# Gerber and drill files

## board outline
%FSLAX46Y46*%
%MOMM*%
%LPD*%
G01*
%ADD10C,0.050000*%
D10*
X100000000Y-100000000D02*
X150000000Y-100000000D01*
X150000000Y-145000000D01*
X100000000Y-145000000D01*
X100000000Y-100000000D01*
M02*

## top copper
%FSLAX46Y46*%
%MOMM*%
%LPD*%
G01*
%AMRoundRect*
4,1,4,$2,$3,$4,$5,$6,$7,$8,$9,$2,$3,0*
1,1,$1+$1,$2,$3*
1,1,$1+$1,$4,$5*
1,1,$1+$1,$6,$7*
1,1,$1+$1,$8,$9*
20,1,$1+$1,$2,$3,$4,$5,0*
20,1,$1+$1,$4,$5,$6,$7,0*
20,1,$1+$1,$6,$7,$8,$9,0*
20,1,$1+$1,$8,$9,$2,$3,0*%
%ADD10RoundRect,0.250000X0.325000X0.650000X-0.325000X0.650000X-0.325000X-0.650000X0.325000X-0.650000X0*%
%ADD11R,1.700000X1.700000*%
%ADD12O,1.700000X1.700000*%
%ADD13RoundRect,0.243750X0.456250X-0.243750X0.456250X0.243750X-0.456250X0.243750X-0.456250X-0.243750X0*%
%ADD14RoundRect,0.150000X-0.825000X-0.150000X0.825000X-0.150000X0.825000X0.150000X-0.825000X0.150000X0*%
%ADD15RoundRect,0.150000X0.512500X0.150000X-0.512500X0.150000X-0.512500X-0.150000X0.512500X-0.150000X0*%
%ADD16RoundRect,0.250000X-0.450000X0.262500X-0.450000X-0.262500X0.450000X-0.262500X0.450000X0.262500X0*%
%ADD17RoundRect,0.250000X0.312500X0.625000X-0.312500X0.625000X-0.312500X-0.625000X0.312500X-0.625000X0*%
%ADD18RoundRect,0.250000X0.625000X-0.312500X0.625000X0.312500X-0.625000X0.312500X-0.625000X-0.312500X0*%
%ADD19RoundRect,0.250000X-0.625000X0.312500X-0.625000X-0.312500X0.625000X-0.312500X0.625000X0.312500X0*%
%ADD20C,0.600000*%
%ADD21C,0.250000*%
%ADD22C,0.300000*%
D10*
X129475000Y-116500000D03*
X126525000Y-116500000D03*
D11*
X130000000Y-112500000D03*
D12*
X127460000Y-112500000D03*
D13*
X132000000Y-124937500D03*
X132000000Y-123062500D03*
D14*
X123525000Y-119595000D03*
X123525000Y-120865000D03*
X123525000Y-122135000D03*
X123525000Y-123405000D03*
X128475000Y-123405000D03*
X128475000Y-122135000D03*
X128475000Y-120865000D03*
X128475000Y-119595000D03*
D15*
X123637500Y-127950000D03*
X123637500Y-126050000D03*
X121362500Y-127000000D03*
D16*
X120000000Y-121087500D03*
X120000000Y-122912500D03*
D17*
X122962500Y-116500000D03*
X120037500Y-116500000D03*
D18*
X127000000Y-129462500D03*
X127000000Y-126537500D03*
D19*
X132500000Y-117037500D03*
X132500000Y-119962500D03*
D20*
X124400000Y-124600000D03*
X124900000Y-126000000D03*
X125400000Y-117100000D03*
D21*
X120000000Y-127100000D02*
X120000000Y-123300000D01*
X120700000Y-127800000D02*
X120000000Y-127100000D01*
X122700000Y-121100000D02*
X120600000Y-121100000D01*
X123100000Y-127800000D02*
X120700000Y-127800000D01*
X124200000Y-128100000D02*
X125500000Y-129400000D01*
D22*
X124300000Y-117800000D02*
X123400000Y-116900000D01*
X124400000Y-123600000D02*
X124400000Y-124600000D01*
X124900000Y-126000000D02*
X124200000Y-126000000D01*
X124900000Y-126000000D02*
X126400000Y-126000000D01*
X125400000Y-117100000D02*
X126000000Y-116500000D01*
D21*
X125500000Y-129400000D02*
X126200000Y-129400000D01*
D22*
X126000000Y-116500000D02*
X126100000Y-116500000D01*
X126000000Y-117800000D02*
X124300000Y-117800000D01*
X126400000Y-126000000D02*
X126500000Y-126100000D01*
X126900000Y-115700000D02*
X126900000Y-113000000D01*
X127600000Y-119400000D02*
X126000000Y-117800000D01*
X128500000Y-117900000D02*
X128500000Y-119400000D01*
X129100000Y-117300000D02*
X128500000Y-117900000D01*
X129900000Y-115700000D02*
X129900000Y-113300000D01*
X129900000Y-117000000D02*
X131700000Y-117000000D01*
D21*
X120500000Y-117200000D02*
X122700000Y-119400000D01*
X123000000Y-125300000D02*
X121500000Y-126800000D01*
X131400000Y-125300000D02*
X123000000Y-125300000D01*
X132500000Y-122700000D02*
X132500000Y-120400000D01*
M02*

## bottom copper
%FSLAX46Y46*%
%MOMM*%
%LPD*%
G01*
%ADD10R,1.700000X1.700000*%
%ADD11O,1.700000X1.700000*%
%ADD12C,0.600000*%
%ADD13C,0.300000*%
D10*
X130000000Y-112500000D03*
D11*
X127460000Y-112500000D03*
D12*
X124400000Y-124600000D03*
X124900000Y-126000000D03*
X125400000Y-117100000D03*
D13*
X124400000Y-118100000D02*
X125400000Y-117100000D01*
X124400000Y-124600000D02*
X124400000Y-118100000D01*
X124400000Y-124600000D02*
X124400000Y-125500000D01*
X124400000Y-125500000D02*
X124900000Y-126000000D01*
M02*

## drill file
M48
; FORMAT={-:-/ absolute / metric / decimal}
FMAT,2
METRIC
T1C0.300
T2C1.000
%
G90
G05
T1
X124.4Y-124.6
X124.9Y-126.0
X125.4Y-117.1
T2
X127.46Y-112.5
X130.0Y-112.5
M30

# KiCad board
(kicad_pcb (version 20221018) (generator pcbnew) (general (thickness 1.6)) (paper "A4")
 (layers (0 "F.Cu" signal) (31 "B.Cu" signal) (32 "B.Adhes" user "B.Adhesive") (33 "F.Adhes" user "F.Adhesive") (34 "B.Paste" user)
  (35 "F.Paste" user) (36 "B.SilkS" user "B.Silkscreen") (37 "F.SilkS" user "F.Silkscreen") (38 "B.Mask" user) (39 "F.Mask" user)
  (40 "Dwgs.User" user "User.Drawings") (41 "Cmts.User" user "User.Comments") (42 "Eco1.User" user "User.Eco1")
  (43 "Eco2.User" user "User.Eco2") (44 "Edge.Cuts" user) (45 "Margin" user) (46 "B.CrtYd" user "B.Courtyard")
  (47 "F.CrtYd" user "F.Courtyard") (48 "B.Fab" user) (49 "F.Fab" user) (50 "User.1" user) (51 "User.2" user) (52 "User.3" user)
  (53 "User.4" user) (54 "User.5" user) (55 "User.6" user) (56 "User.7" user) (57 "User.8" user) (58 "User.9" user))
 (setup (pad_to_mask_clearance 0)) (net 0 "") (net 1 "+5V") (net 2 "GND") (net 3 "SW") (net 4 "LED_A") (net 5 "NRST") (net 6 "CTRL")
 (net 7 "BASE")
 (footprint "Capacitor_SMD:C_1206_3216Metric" (layer "F.Cu") (at 128 116.5 180)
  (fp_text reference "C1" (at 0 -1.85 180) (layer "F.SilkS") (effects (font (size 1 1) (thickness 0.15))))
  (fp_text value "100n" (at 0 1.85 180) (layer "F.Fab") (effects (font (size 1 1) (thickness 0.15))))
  (pad "1" smd roundrect (at -1.475 0 180) (size 1.15 1.8) (layers "F.Cu" "F.Paste" "F.Mask") (roundrect_rratio 0.217391) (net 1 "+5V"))
  (pad "2" smd roundrect (at 1.475 0 180) (size 1.15 1.8) (layers "F.Cu" "F.Paste" "F.Mask") (roundrect_rratio 0.217391) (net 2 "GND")))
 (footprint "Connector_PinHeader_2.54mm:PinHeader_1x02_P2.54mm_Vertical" (layer "F.Cu") (at 130 112.5 -90)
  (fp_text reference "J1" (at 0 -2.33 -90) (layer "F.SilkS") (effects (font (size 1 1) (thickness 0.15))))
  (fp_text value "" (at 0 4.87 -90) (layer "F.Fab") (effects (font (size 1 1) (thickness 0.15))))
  (pad "1" thru_hole rect (at 0 0 270) (size 1.7 1.7) (drill 1) (layers "*.Cu" "*.Mask") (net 1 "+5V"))
  (pad "2" thru_hole oval (at 0 2.54 270) (size 1.7 1.7) (drill 1) (layers "*.Cu" "*.Mask") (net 2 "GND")))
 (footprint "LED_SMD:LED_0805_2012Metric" (layer "F.Cu") (at 132 124 90)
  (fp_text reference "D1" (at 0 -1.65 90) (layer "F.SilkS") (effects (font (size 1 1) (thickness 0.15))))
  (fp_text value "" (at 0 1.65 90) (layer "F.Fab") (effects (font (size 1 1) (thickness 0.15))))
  (pad "1" smd roundrect (at -0.9375 0 90) (size 0.975 1.4) (layers "F.Cu" "F.Paste" "F.Mask") (roundrect_rratio 0.25) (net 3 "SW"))
  (pad "2" smd roundrect (at 0.9375 0 90) (size 0.975 1.4) (layers "F.Cu" "F.Paste" "F.Mask") (roundrect_rratio 0.25) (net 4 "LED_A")))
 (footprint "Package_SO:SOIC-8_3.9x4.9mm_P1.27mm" (layer "F.Cu") (at 126 121.5)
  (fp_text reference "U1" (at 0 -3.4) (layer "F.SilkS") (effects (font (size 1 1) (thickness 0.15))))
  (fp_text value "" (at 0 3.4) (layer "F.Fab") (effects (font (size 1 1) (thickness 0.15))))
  (pad "1" smd roundrect (at -2.475 -1.905) (size 1.95 0.6) (layers "F.Cu" "F.Paste" "F.Mask") (roundrect_rratio 0.25) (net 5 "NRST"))
  (pad "2" smd roundrect (at -2.475 -0.635) (size 1.95 0.6) (layers "F.Cu" "F.Paste" "F.Mask") (roundrect_rratio 0.25) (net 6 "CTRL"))
  (pad "3" smd roundrect (at -2.475 0.635) (size 1.95 0.6) (layers "F.Cu" "F.Paste" "F.Mask") (roundrect_rratio 0.25))
  (pad "4" smd roundrect (at -2.475 1.905) (size 1.95 0.6) (layers "F.Cu" "F.Paste" "F.Mask") (roundrect_rratio 0.25) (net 2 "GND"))
  (pad "5" smd roundrect (at 2.475 1.905) (size 1.95 0.6) (layers "F.Cu" "F.Paste" "F.Mask") (roundrect_rratio 0.25))
  (pad "6" smd roundrect (at 2.475 0.635) (size 1.95 0.6) (layers "F.Cu" "F.Paste" "F.Mask") (roundrect_rratio 0.25))
  (pad "7" smd roundrect (at 2.475 -0.635) (size 1.95 0.6) (layers "F.Cu" "F.Paste" "F.Mask") (roundrect_rratio 0.25))
  (pad "8" smd roundrect (at 2.475 -1.905) (size 1.95 0.6) (layers "F.Cu" "F.Paste" "F.Mask") (roundrect_rratio 0.25) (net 1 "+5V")))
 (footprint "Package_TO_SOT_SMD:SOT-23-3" (layer "F.Cu") (at 122.5 127 180)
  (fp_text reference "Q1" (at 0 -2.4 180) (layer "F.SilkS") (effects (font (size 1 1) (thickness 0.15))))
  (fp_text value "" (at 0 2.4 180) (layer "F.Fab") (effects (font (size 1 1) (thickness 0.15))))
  (pad "1" smd roundrect (at -1.1375 -0.95 180) (size 1.325 0.6) (layers "F.Cu" "F.Paste" "F.Mask") (roundrect_rratio 0.25) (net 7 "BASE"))
  (pad "2" smd roundrect (at -1.1375 0.95 180) (size 1.325 0.6) (layers "F.Cu" "F.Paste" "F.Mask") (roundrect_rratio 0.25) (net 2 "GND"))
  (pad "3" smd roundrect (at 1.1375 0 180) (size 1.325 0.6) (layers "F.Cu" "F.Paste" "F.Mask") (roundrect_rratio 0.25) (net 3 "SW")))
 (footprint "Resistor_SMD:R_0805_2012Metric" (layer "F.Cu") (at 120 122 -90)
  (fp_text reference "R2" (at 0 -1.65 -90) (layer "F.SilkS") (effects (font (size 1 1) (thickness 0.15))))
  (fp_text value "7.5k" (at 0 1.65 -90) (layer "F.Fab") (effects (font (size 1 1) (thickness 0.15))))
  (pad "1" smd roundrect (at -0.9125 0 270) (size 1.025 1.4) (layers "F.Cu" "F.Paste" "F.Mask") (roundrect_rratio 0.243902) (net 6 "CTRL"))
  (pad "2" smd roundrect (at 0.9125 0 270) (size 1.025 1.4) (layers "F.Cu" "F.Paste" "F.Mask") (roundrect_rratio 0.243902) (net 7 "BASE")))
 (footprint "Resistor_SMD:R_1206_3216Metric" (layer "F.Cu") (at 121.5 116.5 180)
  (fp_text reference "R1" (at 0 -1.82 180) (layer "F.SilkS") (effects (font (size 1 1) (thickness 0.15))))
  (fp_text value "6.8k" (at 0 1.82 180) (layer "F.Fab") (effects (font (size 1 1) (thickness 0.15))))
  (pad "1" smd roundrect (at -1.4625 0 180) (size 1.125 1.75) (layers "F.Cu" "F.Paste" "F.Mask") (roundrect_rratio 0.222222) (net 1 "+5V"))
  (pad "2" smd roundrect (at 1.4625 0 180) (size 1.125 1.75) (layers "F.Cu" "F.Paste" "F.Mask") (roundrect_rratio 0.222222) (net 5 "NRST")))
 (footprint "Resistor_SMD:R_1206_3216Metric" (layer "F.Cu") (at 127 128 90)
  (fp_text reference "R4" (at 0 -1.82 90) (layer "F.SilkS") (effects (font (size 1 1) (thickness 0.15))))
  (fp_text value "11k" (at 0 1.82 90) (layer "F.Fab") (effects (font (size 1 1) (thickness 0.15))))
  (pad "1" smd roundrect (at -1.4625 0 90) (size 1.125 1.75) (layers "F.Cu" "F.Paste" "F.Mask") (roundrect_rratio 0.222222) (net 7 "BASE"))
  (pad "2" smd roundrect (at 1.4625 0 90) (size 1.125 1.75) (layers "F.Cu" "F.Paste" "F.Mask") (roundrect_rratio 0.222222) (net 2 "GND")))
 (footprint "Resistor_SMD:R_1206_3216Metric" (layer "F.Cu") (at 132.5 118.5 -90)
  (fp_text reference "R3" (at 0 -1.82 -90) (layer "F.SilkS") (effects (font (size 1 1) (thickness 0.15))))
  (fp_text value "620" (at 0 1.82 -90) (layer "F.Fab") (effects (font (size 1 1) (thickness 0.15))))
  (pad "1" smd roundrect (at -1.4625 0 270) (size 1.125 1.75) (layers "F.Cu" "F.Paste" "F.Mask") (roundrect_rratio 0.222222) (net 1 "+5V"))
  (pad "2" smd roundrect (at 1.4625 0 270) (size 1.125 1.75) (layers "F.Cu" "F.Paste" "F.Mask") (roundrect_rratio 0.222222) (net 4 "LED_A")))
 (gr_rect (start 100 100) (end 150 145) (stroke (width 0.05) (type default)) (fill none) (layer "Edge.Cuts"))
 (segment (start 120 127.1) (end 120 123.3) (width 0.25) (layer "F.Cu") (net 7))
 (segment (start 120.7 127.8) (end 120 127.1) (width 0.25) (layer "F.Cu") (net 7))
 (segment (start 122.7 121.1) (end 120.6 121.1) (width 0.25) (layer "F.Cu") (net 6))
 (segment (start 123.1 127.8) (end 120.7 127.8) (width 0.25) (layer "F.Cu") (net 7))
 (segment (start 124.2 128.1) (end 125.5 129.4) (width 0.25) (layer "F.Cu") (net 7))
 (segment (start 124.3 117.8) (end 123.4 116.9) (width 0.3) (layer "F.Cu") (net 1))
 (segment (start 124.4 123.6) (end 124.4 124.6) (width 0.3) (layer "F.Cu") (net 2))
 (segment (start 124.9 126) (end 124.2 126) (width 0.3) (layer "F.Cu") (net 2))
 (segment (start 124.9 126) (end 126.4 126) (width 0.3) (layer "F.Cu") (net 2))
 (segment (start 125.4 117.1) (end 126 116.5) (width 0.3) (layer "F.Cu") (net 2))
 (segment (start 125.5 129.4) (end 126.2 129.4) (width 0.25) (layer "F.Cu") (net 7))
 (segment (start 126 116.5) (end 126.1 116.5) (width 0.3) (layer "F.Cu") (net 2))
 (segment (start 126 117.8) (end 124.3 117.8) (width 0.3) (layer "F.Cu") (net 1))
 (segment (start 126.4 126) (end 126.5 126.1) (width 0.3) (layer "F.Cu") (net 2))
 (segment (start 126.9 115.7) (end 126.9 113) (width 0.3) (layer "F.Cu") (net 2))
 (segment (start 127.6 119.4) (end 126 117.8) (width 0.3) (layer "F.Cu") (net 1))
 (segment (start 128.5 117.9) (end 128.5 119.4) (width 0.3) (layer "F.Cu") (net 1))
 (segment (start 129.1 117.3) (end 128.5 117.9) (width 0.3) (layer "F.Cu") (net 1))
 (segment (start 129.9 115.7) (end 129.9 113.3) (width 0.3) (layer "F.Cu") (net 1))
 (segment (start 129.9 117) (end 131.7 117) (width 0.3) (layer "F.Cu") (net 1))
 (via (at 124.4 124.6) (size 0.6) (drill 0.3) (layers "F.Cu" "B.Cu") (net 2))
 (via (at 124.9 126) (size 0.6) (drill 0.3) (layers "F.Cu" "B.Cu") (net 2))
 (via (at 125.4 117.1) (size 0.6) (drill 0.3) (layers "F.Cu" "B.Cu") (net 2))
 (segment (start 120.5 117.2) (end 122.7 119.4) (width 0.25) (layer "F.Cu") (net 5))
 (segment (start 123 125.3) (end 121.5 126.8) (width 0.25) (layer "F.Cu") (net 3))
 (segment (start 124.4 118.1) (end 125.4 117.1) (width 0.3) (layer "B.Cu") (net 2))
 (segment (start 124.4 124.6) (end 124.4 118.1) (width 0.3) (layer "B.Cu") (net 2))
 (segment (start 124.4 124.6) (end 124.4 125.5) (width 0.3) (layer "B.Cu") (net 2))
 (segment (start 124.4 125.5) (end 124.9 126) (width 0.3) (layer "B.Cu") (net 2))
 (segment (start 131.4 125.3) (end 123 125.3) (width 0.25) (layer "F.Cu") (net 3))
 (segment (start 132.5 122.7) (end 132.5 120.4) (width 0.25) (layer "F.Cu") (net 4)))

